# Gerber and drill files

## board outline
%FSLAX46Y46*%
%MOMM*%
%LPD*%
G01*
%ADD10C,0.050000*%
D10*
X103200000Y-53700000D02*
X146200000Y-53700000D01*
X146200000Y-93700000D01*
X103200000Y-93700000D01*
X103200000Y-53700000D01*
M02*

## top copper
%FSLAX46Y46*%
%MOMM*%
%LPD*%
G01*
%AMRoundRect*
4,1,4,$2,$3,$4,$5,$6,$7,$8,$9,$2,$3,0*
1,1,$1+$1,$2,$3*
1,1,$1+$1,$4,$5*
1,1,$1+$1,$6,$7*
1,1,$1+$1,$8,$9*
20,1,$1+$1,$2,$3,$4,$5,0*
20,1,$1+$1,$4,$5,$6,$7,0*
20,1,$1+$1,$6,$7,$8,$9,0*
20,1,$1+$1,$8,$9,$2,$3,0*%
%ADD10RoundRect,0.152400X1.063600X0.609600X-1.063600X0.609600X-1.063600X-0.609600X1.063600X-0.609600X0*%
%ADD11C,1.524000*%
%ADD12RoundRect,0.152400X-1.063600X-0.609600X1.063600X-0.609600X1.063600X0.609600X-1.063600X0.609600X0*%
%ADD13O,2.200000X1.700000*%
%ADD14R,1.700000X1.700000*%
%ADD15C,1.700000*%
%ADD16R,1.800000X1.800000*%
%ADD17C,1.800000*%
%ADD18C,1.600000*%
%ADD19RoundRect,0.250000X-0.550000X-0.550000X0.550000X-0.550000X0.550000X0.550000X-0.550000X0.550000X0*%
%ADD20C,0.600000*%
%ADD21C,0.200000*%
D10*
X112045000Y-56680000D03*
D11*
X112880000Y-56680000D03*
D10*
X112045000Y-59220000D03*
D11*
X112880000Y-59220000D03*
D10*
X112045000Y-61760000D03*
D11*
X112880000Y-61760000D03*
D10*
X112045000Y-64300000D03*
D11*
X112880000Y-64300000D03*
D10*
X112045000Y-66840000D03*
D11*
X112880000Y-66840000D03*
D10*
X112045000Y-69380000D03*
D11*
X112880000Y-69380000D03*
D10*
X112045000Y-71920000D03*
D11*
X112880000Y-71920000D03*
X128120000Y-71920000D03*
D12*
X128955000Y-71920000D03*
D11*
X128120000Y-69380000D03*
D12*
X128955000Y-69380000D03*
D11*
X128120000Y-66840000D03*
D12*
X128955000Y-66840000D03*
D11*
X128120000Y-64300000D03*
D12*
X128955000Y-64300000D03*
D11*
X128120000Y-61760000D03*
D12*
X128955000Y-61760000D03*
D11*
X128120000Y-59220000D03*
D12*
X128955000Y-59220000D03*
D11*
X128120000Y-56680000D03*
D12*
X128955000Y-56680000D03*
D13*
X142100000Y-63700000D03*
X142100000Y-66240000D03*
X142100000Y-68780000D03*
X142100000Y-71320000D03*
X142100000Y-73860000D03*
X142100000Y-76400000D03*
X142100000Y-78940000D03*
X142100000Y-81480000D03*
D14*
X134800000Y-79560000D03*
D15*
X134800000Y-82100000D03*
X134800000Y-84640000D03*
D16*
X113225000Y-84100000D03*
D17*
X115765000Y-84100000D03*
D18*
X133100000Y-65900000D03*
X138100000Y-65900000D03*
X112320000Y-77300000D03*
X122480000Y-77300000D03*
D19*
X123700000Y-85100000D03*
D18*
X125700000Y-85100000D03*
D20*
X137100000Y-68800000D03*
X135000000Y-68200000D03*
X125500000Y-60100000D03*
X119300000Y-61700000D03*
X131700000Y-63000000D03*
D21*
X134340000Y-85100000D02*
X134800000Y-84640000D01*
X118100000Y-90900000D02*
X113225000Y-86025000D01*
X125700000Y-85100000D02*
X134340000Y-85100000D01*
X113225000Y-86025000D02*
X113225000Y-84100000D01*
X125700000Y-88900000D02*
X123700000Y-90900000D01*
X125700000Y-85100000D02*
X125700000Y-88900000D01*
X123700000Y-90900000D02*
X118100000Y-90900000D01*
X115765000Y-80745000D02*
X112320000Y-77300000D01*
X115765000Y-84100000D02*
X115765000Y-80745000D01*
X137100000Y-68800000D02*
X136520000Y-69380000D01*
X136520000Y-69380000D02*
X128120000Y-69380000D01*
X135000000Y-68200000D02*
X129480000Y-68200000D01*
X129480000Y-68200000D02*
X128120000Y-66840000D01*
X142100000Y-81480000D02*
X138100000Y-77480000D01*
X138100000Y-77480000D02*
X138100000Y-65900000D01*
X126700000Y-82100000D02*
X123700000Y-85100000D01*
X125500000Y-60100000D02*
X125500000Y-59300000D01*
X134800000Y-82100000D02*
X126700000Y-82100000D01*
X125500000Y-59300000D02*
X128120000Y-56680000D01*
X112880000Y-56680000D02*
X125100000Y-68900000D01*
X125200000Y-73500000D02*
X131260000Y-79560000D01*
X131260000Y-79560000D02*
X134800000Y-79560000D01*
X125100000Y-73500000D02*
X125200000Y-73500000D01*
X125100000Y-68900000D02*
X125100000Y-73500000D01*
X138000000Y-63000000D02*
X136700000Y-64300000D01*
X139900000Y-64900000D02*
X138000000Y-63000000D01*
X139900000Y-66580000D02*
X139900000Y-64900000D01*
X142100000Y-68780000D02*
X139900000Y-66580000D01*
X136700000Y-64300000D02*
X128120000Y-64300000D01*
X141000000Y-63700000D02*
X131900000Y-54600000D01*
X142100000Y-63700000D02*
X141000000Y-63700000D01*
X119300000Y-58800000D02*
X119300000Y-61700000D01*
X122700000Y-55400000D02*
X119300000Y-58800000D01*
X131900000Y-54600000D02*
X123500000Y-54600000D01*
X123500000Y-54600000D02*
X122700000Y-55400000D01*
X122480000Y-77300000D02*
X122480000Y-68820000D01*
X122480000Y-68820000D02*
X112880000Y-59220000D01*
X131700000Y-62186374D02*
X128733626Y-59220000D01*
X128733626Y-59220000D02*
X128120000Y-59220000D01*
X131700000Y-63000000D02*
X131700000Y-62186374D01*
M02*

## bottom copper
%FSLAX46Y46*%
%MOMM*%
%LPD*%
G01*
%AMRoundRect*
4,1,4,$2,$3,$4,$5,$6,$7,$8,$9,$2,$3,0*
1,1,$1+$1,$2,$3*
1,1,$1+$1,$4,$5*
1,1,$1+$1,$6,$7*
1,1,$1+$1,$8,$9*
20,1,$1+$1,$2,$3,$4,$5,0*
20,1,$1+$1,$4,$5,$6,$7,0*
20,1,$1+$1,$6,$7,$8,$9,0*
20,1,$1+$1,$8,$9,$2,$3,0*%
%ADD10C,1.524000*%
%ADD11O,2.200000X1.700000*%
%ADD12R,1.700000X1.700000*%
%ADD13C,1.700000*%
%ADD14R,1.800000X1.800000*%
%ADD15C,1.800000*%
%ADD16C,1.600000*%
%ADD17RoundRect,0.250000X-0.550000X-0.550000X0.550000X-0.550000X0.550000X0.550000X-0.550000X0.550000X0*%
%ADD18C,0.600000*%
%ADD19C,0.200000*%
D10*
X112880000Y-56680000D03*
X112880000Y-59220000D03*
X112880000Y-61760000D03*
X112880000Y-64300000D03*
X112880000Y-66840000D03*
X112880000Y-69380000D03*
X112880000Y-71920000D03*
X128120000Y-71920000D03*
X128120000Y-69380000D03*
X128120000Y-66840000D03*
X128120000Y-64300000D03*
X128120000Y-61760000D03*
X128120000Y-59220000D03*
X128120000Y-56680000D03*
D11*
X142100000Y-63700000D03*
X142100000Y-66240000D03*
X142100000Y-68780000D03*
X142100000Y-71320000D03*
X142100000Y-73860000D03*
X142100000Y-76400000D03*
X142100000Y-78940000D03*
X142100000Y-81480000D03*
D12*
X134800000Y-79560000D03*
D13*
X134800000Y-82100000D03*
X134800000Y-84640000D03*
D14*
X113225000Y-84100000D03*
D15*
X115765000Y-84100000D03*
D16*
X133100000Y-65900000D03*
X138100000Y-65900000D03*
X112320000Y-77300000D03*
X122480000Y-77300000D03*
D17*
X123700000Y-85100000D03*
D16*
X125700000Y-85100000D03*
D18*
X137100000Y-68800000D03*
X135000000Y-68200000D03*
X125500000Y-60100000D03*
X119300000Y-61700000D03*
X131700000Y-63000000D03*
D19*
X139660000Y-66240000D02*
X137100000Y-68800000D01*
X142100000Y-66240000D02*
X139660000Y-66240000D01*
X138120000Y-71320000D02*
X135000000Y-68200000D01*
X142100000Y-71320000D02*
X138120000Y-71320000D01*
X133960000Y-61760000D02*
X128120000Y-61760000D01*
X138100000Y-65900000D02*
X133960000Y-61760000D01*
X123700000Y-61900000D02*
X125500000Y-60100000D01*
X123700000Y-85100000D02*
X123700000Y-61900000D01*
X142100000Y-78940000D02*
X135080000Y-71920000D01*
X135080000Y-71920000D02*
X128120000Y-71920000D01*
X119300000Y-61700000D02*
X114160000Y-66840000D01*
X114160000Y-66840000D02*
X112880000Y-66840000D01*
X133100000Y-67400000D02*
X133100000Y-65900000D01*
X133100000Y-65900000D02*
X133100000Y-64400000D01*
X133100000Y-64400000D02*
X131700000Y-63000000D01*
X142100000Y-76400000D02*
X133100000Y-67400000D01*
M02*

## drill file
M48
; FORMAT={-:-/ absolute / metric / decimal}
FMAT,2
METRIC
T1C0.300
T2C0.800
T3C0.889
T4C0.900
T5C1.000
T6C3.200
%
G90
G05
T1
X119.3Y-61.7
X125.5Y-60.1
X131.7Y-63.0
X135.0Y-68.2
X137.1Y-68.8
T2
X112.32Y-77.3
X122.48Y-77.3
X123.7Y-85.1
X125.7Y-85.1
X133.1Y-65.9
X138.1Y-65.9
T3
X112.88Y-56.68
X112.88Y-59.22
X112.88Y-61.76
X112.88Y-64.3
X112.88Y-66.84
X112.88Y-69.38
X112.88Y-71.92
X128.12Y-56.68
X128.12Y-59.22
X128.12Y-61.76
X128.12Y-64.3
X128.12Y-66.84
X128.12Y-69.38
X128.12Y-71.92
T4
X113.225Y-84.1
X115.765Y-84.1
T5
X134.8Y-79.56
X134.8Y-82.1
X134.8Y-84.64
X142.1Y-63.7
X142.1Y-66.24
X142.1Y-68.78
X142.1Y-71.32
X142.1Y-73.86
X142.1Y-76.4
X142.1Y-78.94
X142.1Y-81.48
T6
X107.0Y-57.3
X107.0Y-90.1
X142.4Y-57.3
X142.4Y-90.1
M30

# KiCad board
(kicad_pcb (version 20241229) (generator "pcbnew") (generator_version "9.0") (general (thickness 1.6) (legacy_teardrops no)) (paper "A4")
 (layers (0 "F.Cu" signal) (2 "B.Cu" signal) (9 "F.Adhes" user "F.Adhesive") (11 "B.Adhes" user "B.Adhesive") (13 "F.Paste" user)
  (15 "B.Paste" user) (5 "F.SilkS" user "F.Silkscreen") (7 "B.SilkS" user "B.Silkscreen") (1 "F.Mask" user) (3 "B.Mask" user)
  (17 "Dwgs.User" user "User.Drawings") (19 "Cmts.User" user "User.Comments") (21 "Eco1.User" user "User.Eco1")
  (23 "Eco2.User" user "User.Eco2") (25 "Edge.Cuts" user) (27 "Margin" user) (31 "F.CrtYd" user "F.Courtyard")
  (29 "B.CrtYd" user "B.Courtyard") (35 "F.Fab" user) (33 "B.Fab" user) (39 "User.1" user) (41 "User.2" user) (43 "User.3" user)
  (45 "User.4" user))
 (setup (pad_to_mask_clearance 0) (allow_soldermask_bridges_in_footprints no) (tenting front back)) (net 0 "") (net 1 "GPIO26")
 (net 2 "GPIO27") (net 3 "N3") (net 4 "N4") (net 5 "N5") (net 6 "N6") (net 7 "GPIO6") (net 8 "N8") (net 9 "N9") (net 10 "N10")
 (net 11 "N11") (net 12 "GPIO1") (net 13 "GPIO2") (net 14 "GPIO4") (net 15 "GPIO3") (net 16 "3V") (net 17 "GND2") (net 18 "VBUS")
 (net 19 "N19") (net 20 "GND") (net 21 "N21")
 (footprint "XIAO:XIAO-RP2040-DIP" (layer "F.Cu") (at 120.5 64.3)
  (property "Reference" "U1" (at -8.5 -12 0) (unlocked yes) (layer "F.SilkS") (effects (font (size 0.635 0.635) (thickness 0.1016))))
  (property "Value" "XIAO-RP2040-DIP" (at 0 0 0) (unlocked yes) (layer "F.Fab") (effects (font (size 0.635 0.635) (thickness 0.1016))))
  (pad "1" smd roundrect (at -8.455 -7.62 180) (size 2.432 1.524) (layers "F.Cu" "F.Mask") (roundrect_rratio 0.1) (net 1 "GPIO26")
   (thermal_bridge_angle 45))
  (pad "1" thru_hole circle (at -7.62 -7.62 180) (size 1.524 1.524) (drill 0.889) (layers "*.Cu" "*.Mask") (remove_unused_layers no)
   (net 1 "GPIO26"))
  (pad "2" smd roundrect (at -8.455 -5.08 180) (size 2.432 1.524) (layers "F.Cu" "F.Mask") (roundrect_rratio 0.1) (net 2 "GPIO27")
   (thermal_bridge_angle 45))
  (pad "2" thru_hole circle (at -7.62 -5.08 180) (size 1.524 1.524) (drill 0.889) (layers "*.Cu" "*.Mask") (remove_unused_layers no)
   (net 2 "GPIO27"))
  (pad "3" smd roundrect (at -8.455 -2.54 180) (size 2.432 1.524) (layers "F.Cu" "F.Mask") (roundrect_rratio 0.1) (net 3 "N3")
   (thermal_bridge_angle 45))
  (pad "3" thru_hole circle (at -7.62 -2.54 180) (size 1.524 1.524) (drill 0.889) (layers "*.Cu" "*.Mask") (remove_unused_layers no)
   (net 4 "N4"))
  (pad "4" smd roundrect (at -8.455 0 180) (size 2.432 1.524) (layers "F.Cu" "F.Mask") (roundrect_rratio 0.1) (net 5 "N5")
   (thermal_bridge_angle 45))
  (pad "4" thru_hole circle (at -7.62 0 180) (size 1.524 1.524) (drill 0.889) (layers "*.Cu" "*.Mask") (remove_unused_layers no)
   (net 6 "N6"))
  (pad "5" smd roundrect (at -8.455 2.54 180) (size 2.432 1.524) (layers "F.Cu" "F.Mask") (roundrect_rratio 0.1) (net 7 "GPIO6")
   (thermal_bridge_angle 45))
  (pad "5" thru_hole circle (at -7.62 2.54 180) (size 1.524 1.524) (drill 0.889) (layers "*.Cu" "*.Mask") (remove_unused_layers no)
   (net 7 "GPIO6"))
  (pad "6" smd roundrect (at -8.455 5.08 180) (size 2.432 1.524) (layers "F.Cu" "F.Mask") (roundrect_rratio 0.1) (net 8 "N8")
   (thermal_bridge_angle 45))
  (pad "6" thru_hole circle (at -7.62 5.08 180) (size 1.524 1.524) (drill 0.889) (layers "*.Cu" "*.Mask") (remove_unused_layers no)
   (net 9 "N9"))
  (pad "7" smd roundrect (at -8.455 7.62 180) (size 2.432 1.524) (layers "F.Cu" "F.Mask") (roundrect_rratio 0.1) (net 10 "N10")
   (thermal_bridge_angle 45))
  (pad "7" thru_hole circle (at -7.62 7.62 180) (size 1.524 1.524) (drill 0.889) (layers "*.Cu" "*.Mask") (remove_unused_layers no)
   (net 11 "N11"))
  (pad "8" thru_hole circle (at 7.62 7.62) (size 1.524 1.524) (drill 0.889) (layers "*.Cu" "*.Mask") (remove_unused_layers no)
   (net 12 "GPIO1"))
  (pad "8" smd roundrect (at 8.455 7.62) (size 2.432 1.524) (layers "F.Cu" "F.Mask") (roundrect_rratio 0.1) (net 12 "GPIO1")
   (thermal_bridge_angle 45))
  (pad "9" thru_hole circle (at 7.62 5.08) (size 1.524 1.524) (drill 0.889) (layers "*.Cu" "*.Mask") (remove_unused_layers no)
   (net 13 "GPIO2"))
  (pad "9" smd roundrect (at 8.455 5.08) (size 2.432 1.524) (layers "F.Cu" "F.Mask") (roundrect_rratio 0.1) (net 13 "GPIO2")
   (thermal_bridge_angle 45))
  (pad "10" thru_hole circle (at 7.62 2.54) (size 1.524 1.524) (drill 0.889) (layers "*.Cu" "*.Mask") (remove_unused_layers no)
   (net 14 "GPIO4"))
  (pad "10" smd roundrect (at 8.455 2.54) (size 2.432 1.524) (layers "F.Cu" "F.Mask") (roundrect_rratio 0.1) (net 14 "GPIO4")
   (thermal_bridge_angle 45))
  (pad "11" thru_hole circle (at 7.62 0) (size 1.524 1.524) (drill 0.889) (layers "*.Cu" "*.Mask") (remove_unused_layers no)
   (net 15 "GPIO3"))
  (pad "11" smd roundrect (at 8.455 0) (size 2.432 1.524) (layers "F.Cu" "F.Mask") (roundrect_rratio 0.1) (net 15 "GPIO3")
   (thermal_bridge_angle 45))
  (pad "12" thru_hole circle (at 7.62 -2.54) (size 1.524 1.524) (drill 0.889) (layers "*.Cu" "*.Mask") (remove_unused_layers no)
   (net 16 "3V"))
  (pad "12" smd roundrect (at 8.455 -2.54) (size 2.432 1.524) (layers "F.Cu" "F.Mask") (roundrect_rratio 0.1) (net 16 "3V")
   (thermal_bridge_angle 45))
  (pad "13" thru_hole circle (at 7.62 -5.08) (size 1.524 1.524) (drill 0.889) (layers "*.Cu" "*.Mask") (remove_unused_layers no)
   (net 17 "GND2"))
  (pad "13" smd roundrect (at 8.455 -5.08) (size 2.432 1.524) (layers "F.Cu" "F.Mask") (roundrect_rratio 0.1) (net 17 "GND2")
   (thermal_bridge_angle 45))
  (pad "14" thru_hole circle (at 7.62 -7.62) (size 1.524 1.524) (drill 0.889) (layers "*.Cu" "*.Mask") (remove_unused_layers no)
   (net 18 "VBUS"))
  (pad "14" smd roundrect (at 8.455 -7.62) (size 2.432 1.524) (layers "F.Cu" "F.Mask") (roundrect_rratio 0.1) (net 18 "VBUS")
   (thermal_bridge_angle 45)))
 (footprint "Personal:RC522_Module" (layer "F.Cu") (at 149.72 68.78 -90)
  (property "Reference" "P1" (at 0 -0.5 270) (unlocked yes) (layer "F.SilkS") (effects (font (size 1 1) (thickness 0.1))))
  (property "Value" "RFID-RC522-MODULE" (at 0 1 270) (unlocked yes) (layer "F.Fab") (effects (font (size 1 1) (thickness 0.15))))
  (pad "1" thru_hole oval (at -5.08 7.62 270) (size 1.7 2.2) (drill 1) (layers "*.Cu" "*.Mask") (remove_unused_layers no) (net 7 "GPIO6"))
  (pad "2" thru_hole oval (at -2.54 7.62 270) (size 1.7 2.2) (drill 1) (layers "*.Cu" "*.Mask") (remove_unused_layers no) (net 13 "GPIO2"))
  (pad "3" thru_hole oval (at 0 7.62 270) (size 1.7 2.2) (drill 1) (layers "*.Cu" "*.Mask") (remove_unused_layers no) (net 15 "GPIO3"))
  (pad "4" thru_hole oval (at 2.54 7.62 270) (size 1.7 2.2) (drill 1) (layers "*.Cu" "*.Mask") (remove_unused_layers no) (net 14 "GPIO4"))
  (pad "5" thru_hole oval (at 5.08 7.62 270) (size 1.7 2.2) (drill 1) (layers "*.Cu" "*.Mask") (remove_unused_layers no) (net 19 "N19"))
  (pad "6" thru_hole oval (at 7.62 7.62 270) (size 1.7 2.2) (drill 1) (layers "*.Cu" "*.Mask") (remove_unused_layers no) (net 17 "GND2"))
  (pad "7" thru_hole oval (at 10.16 7.62 270) (size 1.7 2.2) (drill 1) (layers "*.Cu" "*.Mask") (remove_unused_layers no) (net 12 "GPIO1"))
  (pad "8" thru_hole oval (at 12.7 7.62 270) (size 1.7 2.2) (drill 1) (layers "*.Cu" "*.Mask") (remove_unused_layers no) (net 16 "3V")))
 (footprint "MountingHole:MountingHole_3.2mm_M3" (layer "F.Cu") (at 107 90.1)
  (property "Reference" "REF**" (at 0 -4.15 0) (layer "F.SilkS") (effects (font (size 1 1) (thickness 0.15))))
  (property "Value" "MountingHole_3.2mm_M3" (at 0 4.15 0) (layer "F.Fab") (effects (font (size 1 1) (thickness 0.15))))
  (pad "" np_thru_hole circle (at 0 0) (size 3.2 3.2) (drill 3.2) (layers "*.Cu" "*.Mask")))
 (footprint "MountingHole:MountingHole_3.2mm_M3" (layer "F.Cu") (at 107 57.3)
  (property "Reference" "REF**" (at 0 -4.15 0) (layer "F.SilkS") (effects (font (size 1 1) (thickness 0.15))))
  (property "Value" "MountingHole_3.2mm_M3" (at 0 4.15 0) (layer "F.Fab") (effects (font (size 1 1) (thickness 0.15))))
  (pad "" np_thru_hole circle (at 0 0) (size 3.2 3.2) (drill 3.2) (layers "*.Cu" "*.Mask")))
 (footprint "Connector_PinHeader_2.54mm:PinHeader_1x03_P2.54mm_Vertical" (layer "F.Cu") (at 134.8 79.56)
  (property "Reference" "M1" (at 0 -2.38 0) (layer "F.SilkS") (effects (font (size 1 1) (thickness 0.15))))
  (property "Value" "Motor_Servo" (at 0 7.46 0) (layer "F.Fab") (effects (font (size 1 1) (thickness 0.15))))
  (pad "1" thru_hole rect (at 0 0) (size 1.7 1.7) (drill 1) (layers "*.Cu" "*.Mask") (remove_unused_layers no) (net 1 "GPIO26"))
  (pad "2" thru_hole circle (at 0 2.54) (size 1.7 1.7) (drill 1) (layers "*.Cu" "*.Mask") (remove_unused_layers no) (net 18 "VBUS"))
  (pad "3" thru_hole circle (at 0 5.08) (size 1.7 1.7) (drill 1) (layers "*.Cu" "*.Mask") (remove_unused_layers no) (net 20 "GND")))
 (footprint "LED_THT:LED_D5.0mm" (layer "F.Cu") (at 113.225 84.1)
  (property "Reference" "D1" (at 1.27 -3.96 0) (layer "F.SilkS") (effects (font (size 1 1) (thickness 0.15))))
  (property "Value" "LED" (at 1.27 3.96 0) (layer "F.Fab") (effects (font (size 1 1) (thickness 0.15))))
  (pad "1" thru_hole rect (at 0 0) (size 1.8 1.8) (drill 0.9) (layers "*.Cu" "*.Mask") (remove_unused_layers no) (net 20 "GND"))
  (pad "2" thru_hole circle (at 2.54 0) (size 1.8 1.8) (drill 0.9) (layers "*.Cu" "*.Mask") (remove_unused_layers no) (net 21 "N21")))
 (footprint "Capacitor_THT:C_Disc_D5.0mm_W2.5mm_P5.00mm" (layer "F.Cu") (at 133.1 65.9)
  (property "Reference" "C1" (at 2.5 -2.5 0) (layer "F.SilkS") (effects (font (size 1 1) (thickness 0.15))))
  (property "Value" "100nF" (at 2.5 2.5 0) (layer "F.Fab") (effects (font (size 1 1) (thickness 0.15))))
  (pad "1" thru_hole circle (at 0 0) (size 1.6 1.6) (drill 0.8) (layers "*.Cu" "*.Mask") (remove_unused_layers no) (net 17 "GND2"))
  (pad "2" thru_hole circle (at 5 0) (size 1.6 1.6) (drill 0.8) (layers "*.Cu" "*.Mask") (remove_unused_layers no) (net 16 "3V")))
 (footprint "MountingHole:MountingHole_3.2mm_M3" (layer "F.Cu") (at 142.4 57.3)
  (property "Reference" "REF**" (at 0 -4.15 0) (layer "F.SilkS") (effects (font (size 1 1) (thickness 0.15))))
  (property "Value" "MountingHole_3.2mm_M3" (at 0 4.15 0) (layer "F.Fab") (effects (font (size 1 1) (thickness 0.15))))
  (pad "" np_thru_hole circle (at 0 0) (size 3.2 3.2) (drill 3.2) (layers "*.Cu" "*.Mask")))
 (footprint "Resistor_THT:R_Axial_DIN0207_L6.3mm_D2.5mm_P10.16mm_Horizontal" (layer "F.Cu") (at 112.32 77.3)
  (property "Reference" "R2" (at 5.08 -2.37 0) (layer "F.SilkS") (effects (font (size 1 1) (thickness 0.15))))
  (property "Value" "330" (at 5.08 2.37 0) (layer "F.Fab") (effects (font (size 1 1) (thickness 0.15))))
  (pad "1" thru_hole circle (at 0 0) (size 1.6 1.6) (drill 0.8) (layers "*.Cu" "*.Mask") (remove_unused_layers no) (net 21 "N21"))
  (pad "2" thru_hole circle (at 10.16 0) (size 1.6 1.6) (drill 0.8) (layers "*.Cu" "*.Mask") (remove_unused_layers no) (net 2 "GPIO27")))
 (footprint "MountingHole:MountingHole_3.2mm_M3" (layer "F.Cu") (at 142.4 90.1)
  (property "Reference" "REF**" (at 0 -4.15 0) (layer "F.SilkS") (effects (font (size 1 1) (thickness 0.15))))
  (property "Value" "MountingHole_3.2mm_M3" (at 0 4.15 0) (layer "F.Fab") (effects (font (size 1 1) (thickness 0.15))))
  (pad "" np_thru_hole circle (at 0 0) (size 3.2 3.2) (drill 3.2) (layers "*.Cu" "*.Mask")))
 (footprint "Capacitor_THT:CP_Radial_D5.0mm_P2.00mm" (layer "F.Cu") (at 123.7 85.1)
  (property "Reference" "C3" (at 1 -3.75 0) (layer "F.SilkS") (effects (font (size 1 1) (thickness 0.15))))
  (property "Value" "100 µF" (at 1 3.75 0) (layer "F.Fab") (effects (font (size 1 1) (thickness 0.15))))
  (pad "1" thru_hole roundrect (at 0 0) (size 1.6 1.6) (drill 0.8) (layers "*.Cu" "*.Mask") (remove_unused_layers no)
   (roundrect_rratio 0.15625) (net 18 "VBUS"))
  (pad "2" thru_hole circle (at 2 0) (size 1.6 1.6) (drill 0.8) (layers "*.Cu" "*.Mask") (remove_unused_layers no) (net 20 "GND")))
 (gr_rect (start 103.2 53.7) (end 146.2 93.7) (stroke (width 0.05) (type default)) (fill no) (layer "Edge.Cuts"))
 (segment (start 134.34 85.1) (end 134.8 84.64) (width 0.2) (layer "F.Cu") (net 20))
 (segment (start 118.1 90.9) (end 113.225 86.025) (width 0.2) (layer "F.Cu") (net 20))
 (segment (start 125.7 85.1) (end 134.34 85.1) (width 0.2) (layer "F.Cu") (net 20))
 (segment (start 113.225 86.025) (end 113.225 84.1) (width 0.2) (layer "F.Cu") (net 20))
 (segment (start 125.7 88.9) (end 123.7 90.9) (width 0.2) (layer "F.Cu") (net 20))
 (segment (start 125.7 85.1) (end 125.7 88.9) (width 0.2) (layer "F.Cu") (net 20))
 (segment (start 123.7 90.9) (end 118.1 90.9) (width 0.2) (layer "F.Cu") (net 20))
 (segment (start 115.765 80.745) (end 112.32 77.3) (width 0.2) (layer "F.Cu") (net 21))
 (segment (start 115.765 84.1) (end 115.765 80.745) (width 0.2) (layer "F.Cu") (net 21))
 (segment (start 137.1 68.8) (end 136.52 69.38) (width 0.2) (layer "F.Cu") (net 13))
 (segment (start 136.52 69.38) (end 128.12 69.38) (width 0.2) (layer "F.Cu") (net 13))
 (via (at 137.1 68.8) (size 0.6) (drill 0.3) (layers "F.Cu" "B.Cu") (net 13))
 (segment (start 139.66 66.24) (end 137.1 68.8) (width 0.2) (layer "B.Cu") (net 13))
 (segment (start 142.1 66.24) (end 139.66 66.24) (width 0.2) (layer "B.Cu") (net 13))
 (segment (start 135 68.2) (end 129.48 68.2) (width 0.2) (layer "F.Cu") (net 14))
 (segment (start 129.48 68.2) (end 128.12 66.84) (width 0.2) (layer "F.Cu") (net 14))
 (via (at 135 68.2) (size 0.6) (drill 0.3) (layers "F.Cu" "B.Cu") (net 14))
 (segment (start 138.12 71.32) (end 135 68.2) (width 0.2) (layer "B.Cu") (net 14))
 (segment (start 142.1 71.32) (end 138.12 71.32) (width 0.2) (layer "B.Cu") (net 14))
 (segment (start 142.1 81.48) (end 138.1 77.48) (width 0.2) (layer "F.Cu") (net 16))
 (segment (start 138.1 77.48) (end 138.1 65.9) (width 0.2) (layer "F.Cu") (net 16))
 (segment (start 133.96 61.76) (end 128.12 61.76) (width 0.2) (layer "B.Cu") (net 16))
 (segment (start 138.1 65.9) (end 133.96 61.76) (width 0.2) (layer "B.Cu") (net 16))
 (segment (start 126.7 82.1) (end 123.7 85.1) (width 0.2) (layer "F.Cu") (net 18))
 (segment (start 125.5 60.1) (end 125.5 59.3) (width 0.2) (layer "F.Cu") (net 18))
 (segment (start 134.8 82.1) (end 126.7 82.1) (width 0.2) (layer "F.Cu") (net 18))
 (segment (start 125.5 59.3) (end 128.12 56.68) (width 0.2) (layer "F.Cu") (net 18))
 (via (at 125.5 60.1) (size 0.6) (drill 0.3) (layers "F.Cu" "B.Cu") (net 18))
 (segment (start 123.7 61.9) (end 125.5 60.1) (width 0.2) (layer "B.Cu") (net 18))
 (segment (start 123.7 85.1) (end 123.7 61.9) (width 0.2) (layer "B.Cu") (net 18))
 (segment (start 112.88 56.68) (end 125.1 68.9) (width 0.2) (layer "F.Cu") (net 1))
 (segment (start 125.2 73.5) (end 131.26 79.56) (width 0.2) (layer "F.Cu") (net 1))
 (segment (start 131.26 79.56) (end 134.8 79.56) (width 0.2) (layer "F.Cu") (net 1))
 (segment (start 125.1 73.5) (end 125.2 73.5) (width 0.2) (layer "F.Cu") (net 1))
 (segment (start 125.1 68.9) (end 125.1 73.5) (width 0.2) (layer "F.Cu") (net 1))
 (segment (start 142.1 78.94) (end 135.08 71.92) (width 0.2) (layer "B.Cu") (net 12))
 (segment (start 135.08 71.92) (end 128.12 71.92) (width 0.2) (layer "B.Cu") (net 12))
 (segment (start 138 63) (end 136.7 64.3) (width 0.2) (layer "F.Cu") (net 15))
 (segment (start 139.9 64.9) (end 138 63) (width 0.2) (layer "F.Cu") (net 15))
 (segment (start 139.9 66.58) (end 139.9 64.9) (width 0.2) (layer "F.Cu") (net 15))
 (segment (start 142.1 68.78) (end 139.9 66.58) (width 0.2) (layer "F.Cu") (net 15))
 (segment (start 136.7 64.3) (end 128.12 64.3) (width 0.2) (layer "F.Cu") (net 15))
 (segment (start 141 63.7) (end 131.9 54.6) (width 0.2) (layer "F.Cu") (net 7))
 (segment (start 142.1 63.7) (end 141 63.7) (width 0.2) (layer "F.Cu") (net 7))
 (segment (start 119.3 58.8) (end 119.3 61.7) (width 0.2) (layer "F.Cu") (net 7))
 (segment (start 122.7 55.4) (end 119.3 58.8) (width 0.2) (layer "F.Cu") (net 7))
 (segment (start 131.9 54.6) (end 123.5 54.6) (width 0.2) (layer "F.Cu") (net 7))
 (segment (start 123.5 54.6) (end 122.7 55.4) (width 0.2) (layer "F.Cu") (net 7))
 (via (at 119.3 61.7) (size 0.6) (drill 0.3) (layers "F.Cu" "B.Cu") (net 7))
 (segment (start 119.3 61.7) (end 114.16 66.84) (width 0.2) (layer "B.Cu") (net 7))
 (segment (start 114.16 66.84) (end 112.88 66.84) (width 0.2) (layer "B.Cu") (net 7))
 (segment (start 122.48 77.3) (end 122.48 68.82) (width 0.2) (layer "F.Cu") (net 2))
 (segment (start 122.48 68.82) (end 112.88 59.22) (width 0.2) (layer "F.Cu") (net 2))
 (segment (start 131.7 62.186374) (end 128.733626 59.22) (width 0.2) (layer "F.Cu") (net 17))
 (segment (start 128.733626 59.22) (end 128.12 59.22) (width 0.2) (layer "F.Cu") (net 17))
 (segment (start 131.7 63) (end 131.7 62.186374) (width 0.2) (layer "F.Cu") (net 17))
 (via (at 131.7 63) (size 0.6) (drill 0.3) (layers "F.Cu" "B.Cu") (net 17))
 (segment (start 133.1 67.4) (end 133.1 65.9) (width 0.2) (layer "B.Cu") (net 17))
 (segment (start 133.1 65.9) (end 133.1 64.4) (width 0.2) (layer "B.Cu") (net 17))
 (segment (start 133.1 64.4) (end 131.7 63) (width 0.2) (layer "B.Cu") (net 17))
 (segment (start 142.1 76.4) (end 133.1 67.4) (width 0.2) (layer "B.Cu") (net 17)))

